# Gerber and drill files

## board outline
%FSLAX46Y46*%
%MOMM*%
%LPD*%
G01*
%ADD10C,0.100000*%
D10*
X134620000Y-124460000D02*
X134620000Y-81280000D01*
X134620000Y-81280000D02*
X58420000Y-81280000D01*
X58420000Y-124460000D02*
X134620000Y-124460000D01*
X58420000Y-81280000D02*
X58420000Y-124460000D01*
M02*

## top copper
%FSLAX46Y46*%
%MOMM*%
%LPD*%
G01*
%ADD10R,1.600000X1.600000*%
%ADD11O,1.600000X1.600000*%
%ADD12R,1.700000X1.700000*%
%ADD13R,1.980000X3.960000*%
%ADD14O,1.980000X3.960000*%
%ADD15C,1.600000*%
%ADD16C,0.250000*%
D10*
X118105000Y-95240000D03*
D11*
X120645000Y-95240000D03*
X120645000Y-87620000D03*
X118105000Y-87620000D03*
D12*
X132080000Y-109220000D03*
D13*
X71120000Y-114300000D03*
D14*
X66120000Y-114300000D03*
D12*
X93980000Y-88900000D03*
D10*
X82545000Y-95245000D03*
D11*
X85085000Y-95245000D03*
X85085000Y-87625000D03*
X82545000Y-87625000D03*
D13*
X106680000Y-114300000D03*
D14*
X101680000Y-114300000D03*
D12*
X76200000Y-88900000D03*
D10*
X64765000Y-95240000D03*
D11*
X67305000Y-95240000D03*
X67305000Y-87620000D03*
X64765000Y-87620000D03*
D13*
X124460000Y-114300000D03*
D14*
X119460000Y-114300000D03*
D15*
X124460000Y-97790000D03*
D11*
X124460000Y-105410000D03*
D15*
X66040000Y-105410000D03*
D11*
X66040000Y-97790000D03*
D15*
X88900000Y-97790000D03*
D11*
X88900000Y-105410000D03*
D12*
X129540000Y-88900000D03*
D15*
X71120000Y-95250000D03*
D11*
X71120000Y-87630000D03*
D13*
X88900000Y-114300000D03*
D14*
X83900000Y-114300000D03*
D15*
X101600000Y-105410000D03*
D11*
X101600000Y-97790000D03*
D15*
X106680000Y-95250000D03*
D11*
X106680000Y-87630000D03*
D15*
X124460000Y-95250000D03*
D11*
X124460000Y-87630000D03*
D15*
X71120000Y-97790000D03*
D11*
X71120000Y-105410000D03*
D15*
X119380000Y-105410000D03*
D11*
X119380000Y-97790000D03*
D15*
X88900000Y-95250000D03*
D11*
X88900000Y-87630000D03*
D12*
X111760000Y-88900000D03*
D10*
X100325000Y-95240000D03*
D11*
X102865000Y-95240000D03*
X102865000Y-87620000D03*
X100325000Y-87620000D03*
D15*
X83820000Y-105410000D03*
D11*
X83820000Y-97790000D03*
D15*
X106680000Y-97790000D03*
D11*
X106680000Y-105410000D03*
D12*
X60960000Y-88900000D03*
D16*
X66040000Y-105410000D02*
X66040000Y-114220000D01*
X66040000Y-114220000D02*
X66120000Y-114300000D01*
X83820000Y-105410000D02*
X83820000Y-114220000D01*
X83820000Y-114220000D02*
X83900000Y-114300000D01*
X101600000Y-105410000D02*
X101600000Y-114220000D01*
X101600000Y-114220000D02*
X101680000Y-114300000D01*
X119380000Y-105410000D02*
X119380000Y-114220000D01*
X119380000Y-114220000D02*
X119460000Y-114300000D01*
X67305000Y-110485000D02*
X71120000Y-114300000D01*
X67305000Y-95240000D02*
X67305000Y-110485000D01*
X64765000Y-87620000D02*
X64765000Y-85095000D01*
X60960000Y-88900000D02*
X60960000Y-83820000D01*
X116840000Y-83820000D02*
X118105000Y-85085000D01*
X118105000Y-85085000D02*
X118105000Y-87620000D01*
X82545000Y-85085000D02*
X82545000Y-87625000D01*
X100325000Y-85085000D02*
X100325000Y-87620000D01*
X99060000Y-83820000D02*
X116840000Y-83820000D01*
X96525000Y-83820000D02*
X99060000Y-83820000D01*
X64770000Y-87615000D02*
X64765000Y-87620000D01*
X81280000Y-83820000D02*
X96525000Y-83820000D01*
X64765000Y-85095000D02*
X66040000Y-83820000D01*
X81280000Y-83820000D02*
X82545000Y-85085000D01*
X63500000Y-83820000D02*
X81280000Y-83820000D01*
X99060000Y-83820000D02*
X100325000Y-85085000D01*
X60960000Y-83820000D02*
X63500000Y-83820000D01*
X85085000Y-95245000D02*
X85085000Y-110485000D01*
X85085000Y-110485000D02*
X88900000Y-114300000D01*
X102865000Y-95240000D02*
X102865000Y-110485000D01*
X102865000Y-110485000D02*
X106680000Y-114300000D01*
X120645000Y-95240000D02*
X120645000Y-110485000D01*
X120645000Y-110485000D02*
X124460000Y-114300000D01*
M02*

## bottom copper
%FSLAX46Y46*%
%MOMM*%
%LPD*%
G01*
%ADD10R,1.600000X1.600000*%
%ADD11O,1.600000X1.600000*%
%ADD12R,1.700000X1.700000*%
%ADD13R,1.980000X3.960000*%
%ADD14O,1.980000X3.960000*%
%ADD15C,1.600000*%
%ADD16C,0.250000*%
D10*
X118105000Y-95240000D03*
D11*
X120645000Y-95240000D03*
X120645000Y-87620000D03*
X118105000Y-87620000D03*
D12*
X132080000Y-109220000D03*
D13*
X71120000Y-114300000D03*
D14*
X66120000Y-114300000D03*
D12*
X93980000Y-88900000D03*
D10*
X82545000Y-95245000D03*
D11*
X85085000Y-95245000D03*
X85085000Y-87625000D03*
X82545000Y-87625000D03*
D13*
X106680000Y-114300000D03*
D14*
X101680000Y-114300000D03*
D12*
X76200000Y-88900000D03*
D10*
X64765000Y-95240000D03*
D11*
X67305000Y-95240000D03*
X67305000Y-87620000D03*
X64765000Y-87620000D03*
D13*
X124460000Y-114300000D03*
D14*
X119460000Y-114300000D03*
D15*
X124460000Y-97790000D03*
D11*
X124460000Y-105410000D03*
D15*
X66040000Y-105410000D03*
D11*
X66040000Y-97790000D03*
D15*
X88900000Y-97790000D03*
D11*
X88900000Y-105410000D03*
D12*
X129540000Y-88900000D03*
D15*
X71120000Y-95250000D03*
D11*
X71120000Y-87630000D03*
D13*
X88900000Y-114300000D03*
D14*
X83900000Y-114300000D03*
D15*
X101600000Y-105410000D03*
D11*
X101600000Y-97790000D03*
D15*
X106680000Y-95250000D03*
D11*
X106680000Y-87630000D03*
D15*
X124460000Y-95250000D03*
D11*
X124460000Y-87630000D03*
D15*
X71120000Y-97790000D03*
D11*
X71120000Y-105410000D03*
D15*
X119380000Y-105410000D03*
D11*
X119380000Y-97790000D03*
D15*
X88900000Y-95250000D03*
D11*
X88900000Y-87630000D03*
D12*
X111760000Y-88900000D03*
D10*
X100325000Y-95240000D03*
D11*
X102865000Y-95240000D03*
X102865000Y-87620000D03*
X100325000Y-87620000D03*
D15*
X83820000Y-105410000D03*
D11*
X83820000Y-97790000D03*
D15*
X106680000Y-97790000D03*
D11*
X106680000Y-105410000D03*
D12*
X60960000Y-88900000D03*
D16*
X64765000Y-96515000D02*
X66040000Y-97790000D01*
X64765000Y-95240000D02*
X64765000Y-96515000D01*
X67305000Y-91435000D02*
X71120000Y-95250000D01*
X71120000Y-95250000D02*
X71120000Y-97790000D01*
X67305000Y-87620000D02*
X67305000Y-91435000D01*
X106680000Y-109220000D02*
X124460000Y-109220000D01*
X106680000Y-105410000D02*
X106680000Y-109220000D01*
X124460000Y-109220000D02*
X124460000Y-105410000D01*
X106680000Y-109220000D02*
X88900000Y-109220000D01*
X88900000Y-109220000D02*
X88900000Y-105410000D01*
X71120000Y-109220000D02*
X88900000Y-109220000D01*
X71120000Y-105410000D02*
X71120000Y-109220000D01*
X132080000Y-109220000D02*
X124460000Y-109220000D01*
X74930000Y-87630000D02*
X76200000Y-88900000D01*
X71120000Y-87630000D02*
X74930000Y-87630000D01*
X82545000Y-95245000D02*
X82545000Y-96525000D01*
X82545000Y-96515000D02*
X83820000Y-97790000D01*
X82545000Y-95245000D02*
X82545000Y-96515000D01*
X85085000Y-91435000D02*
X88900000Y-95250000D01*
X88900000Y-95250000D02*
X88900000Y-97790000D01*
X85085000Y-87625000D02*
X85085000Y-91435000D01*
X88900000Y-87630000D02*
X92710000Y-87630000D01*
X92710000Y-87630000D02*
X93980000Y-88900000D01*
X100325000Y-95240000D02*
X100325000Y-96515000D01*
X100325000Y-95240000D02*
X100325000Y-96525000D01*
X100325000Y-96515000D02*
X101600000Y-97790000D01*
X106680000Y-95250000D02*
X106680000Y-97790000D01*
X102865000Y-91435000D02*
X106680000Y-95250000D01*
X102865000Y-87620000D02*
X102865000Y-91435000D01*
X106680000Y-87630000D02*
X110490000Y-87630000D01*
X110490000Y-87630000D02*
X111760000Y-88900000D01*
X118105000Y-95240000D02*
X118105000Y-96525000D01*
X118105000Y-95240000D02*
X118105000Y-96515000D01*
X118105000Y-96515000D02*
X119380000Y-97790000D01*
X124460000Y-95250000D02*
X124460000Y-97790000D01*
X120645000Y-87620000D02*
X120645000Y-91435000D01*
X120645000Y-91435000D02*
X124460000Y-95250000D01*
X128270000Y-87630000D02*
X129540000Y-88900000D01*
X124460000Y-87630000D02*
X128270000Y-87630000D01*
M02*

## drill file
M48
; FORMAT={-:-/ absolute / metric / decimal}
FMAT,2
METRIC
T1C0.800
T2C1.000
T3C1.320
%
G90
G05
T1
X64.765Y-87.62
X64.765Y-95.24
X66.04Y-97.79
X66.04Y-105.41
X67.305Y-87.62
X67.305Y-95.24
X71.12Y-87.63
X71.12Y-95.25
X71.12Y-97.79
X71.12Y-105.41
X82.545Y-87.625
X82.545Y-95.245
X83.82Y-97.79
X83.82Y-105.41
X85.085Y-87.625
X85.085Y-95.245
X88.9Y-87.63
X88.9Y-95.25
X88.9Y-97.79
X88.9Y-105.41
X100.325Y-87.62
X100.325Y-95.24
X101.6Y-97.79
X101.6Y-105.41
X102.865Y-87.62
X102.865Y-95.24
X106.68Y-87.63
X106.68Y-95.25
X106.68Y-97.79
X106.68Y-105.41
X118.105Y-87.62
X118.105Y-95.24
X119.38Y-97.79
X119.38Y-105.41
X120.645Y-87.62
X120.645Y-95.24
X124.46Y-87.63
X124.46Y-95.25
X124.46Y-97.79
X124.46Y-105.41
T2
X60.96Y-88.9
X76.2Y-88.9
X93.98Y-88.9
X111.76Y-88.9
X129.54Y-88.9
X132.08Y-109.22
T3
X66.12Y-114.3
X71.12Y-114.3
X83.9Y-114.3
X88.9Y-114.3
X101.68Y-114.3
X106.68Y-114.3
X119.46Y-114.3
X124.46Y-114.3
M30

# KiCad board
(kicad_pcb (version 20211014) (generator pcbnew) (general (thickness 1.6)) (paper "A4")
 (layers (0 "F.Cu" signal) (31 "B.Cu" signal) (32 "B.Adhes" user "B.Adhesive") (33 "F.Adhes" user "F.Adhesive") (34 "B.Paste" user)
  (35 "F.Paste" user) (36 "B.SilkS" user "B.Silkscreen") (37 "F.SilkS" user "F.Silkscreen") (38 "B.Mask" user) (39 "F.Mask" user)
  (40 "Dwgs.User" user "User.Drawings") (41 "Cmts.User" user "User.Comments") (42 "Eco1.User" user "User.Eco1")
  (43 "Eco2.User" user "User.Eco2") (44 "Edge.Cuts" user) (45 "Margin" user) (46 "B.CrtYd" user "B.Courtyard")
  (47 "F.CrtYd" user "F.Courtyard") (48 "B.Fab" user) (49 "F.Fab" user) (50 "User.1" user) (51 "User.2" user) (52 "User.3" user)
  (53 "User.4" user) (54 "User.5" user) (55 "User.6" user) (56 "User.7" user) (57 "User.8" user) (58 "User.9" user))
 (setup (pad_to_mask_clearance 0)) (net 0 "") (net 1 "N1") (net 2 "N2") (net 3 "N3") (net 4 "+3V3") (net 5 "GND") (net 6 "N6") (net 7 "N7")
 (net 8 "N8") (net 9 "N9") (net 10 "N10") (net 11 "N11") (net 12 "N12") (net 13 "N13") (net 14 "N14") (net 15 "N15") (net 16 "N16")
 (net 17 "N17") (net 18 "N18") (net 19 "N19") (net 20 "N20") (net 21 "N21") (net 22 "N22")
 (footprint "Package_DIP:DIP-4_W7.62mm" (layer "F.Cu") (at 118.105 95.24 90)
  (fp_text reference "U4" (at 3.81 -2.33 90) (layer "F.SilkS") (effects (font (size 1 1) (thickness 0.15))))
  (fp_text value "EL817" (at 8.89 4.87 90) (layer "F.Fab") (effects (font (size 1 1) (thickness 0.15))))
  (pad "1" thru_hole rect (at 0 0 90) (size 1.6 1.6) (drill 0.8) (layers *.Cu *.Mask) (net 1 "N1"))
  (pad "2" thru_hole oval (at 0 2.54 90) (size 1.6 1.6) (drill 0.8) (layers *.Cu *.Mask) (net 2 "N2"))
  (pad "3" thru_hole oval (at 7.62 2.54 90) (size 1.6 1.6) (drill 0.8) (layers *.Cu *.Mask) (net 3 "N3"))
  (pad "4" thru_hole oval (at 7.62 0 90) (size 1.6 1.6) (drill 0.8) (layers *.Cu *.Mask) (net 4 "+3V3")))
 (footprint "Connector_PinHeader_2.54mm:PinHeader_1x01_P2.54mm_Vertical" (layer "F.Cu") (at 132.08 109.22)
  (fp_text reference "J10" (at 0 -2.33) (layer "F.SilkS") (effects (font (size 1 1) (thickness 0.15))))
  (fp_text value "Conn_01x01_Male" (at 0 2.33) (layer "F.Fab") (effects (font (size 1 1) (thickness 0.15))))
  (pad "1" thru_hole rect (at 0 0) (size 1.7 1.7) (drill 1) (layers *.Cu *.Mask) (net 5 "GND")))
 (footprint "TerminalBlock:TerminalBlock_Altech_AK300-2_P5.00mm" (layer "F.Cu") (at 71.12 114.3 180)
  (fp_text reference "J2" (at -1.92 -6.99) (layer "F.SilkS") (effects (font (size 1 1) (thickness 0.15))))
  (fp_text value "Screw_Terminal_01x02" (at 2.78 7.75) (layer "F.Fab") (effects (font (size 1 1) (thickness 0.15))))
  (pad "1" thru_hole rect (at 0 0 180) (size 1.98 3.96) (drill 1.32) (layers *.Cu *.Mask) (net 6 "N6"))
  (pad "2" thru_hole oval (at 5 0 180) (size 1.98 3.96) (drill 1.32) (layers *.Cu *.Mask) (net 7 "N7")))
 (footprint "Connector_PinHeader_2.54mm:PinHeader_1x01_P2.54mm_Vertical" (layer "F.Cu") (at 93.98 88.9)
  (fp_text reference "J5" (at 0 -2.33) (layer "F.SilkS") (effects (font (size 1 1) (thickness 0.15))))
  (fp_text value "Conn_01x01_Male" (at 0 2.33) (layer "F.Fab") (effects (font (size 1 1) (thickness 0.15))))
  (pad "1" thru_hole rect (at 0 0) (size 1.7 1.7) (drill 1) (layers *.Cu *.Mask) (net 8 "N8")))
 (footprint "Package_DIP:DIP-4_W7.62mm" (layer "F.Cu") (at 82.545 95.245 90)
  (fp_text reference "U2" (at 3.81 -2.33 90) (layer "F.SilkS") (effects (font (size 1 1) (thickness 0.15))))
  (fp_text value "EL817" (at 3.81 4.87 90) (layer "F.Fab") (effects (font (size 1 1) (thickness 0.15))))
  (pad "1" thru_hole rect (at 0 0 90) (size 1.6 1.6) (drill 0.8) (layers *.Cu *.Mask) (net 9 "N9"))
  (pad "2" thru_hole oval (at 0 2.54 90) (size 1.6 1.6) (drill 0.8) (layers *.Cu *.Mask) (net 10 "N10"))
  (pad "3" thru_hole oval (at 7.62 2.54 90) (size 1.6 1.6) (drill 0.8) (layers *.Cu *.Mask) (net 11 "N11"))
  (pad "4" thru_hole oval (at 7.62 0 90) (size 1.6 1.6) (drill 0.8) (layers *.Cu *.Mask) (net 4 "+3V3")))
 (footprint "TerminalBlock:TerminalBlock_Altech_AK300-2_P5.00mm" (layer "F.Cu") (at 106.68 114.3 180)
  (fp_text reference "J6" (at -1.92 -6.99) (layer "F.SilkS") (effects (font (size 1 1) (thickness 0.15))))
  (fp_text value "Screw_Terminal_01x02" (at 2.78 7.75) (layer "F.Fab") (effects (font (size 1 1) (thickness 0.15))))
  (pad "1" thru_hole rect (at 0 0 180) (size 1.98 3.96) (drill 1.32) (layers *.Cu *.Mask) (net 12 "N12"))
  (pad "2" thru_hole oval (at 5 0 180) (size 1.98 3.96) (drill 1.32) (layers *.Cu *.Mask) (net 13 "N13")))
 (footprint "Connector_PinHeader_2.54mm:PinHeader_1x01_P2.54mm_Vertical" (layer "F.Cu") (at 76.2 88.9)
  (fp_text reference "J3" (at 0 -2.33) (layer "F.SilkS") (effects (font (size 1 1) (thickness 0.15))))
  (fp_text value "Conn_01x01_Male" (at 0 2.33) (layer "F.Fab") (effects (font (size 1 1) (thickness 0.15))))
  (pad "1" thru_hole rect (at 0 0) (size 1.7 1.7) (drill 1) (layers *.Cu *.Mask) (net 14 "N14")))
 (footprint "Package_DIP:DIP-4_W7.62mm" (layer "F.Cu") (at 64.765 95.24 90)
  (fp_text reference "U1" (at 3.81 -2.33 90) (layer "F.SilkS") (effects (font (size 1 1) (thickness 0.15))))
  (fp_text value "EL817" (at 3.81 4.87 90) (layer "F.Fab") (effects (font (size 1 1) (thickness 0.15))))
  (pad "1" thru_hole rect (at 0 0 90) (size 1.6 1.6) (drill 0.8) (layers *.Cu *.Mask) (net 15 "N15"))
  (pad "2" thru_hole oval (at 0 2.54 90) (size 1.6 1.6) (drill 0.8) (layers *.Cu *.Mask) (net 6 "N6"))
  (pad "3" thru_hole oval (at 7.62 2.54 90) (size 1.6 1.6) (drill 0.8) (layers *.Cu *.Mask) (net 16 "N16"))
  (pad "4" thru_hole oval (at 7.62 0 90) (size 1.6 1.6) (drill 0.8) (layers *.Cu *.Mask) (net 4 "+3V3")))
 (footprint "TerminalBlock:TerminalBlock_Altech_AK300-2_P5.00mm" (layer "F.Cu") (at 124.46 114.3 180)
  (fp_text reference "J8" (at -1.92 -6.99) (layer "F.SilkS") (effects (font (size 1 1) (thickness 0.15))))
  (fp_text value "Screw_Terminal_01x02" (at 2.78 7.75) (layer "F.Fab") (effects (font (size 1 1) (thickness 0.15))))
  (pad "1" thru_hole rect (at 0 0 180) (size 1.98 3.96) (drill 1.32) (layers *.Cu *.Mask) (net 2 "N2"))
  (pad "2" thru_hole oval (at 5 0 180) (size 1.98 3.96) (drill 1.32) (layers *.Cu *.Mask) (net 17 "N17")))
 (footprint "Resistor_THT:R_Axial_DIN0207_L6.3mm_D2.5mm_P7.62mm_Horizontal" (layer "F.Cu") (at 124.46 97.79 -90)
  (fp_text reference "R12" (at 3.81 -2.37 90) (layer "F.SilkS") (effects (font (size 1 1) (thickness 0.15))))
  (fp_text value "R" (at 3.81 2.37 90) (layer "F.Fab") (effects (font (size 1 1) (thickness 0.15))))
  (pad "1" thru_hole circle (at 0 0 270) (size 1.6 1.6) (drill 0.8) (layers *.Cu *.Mask) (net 3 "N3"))
  (pad "2" thru_hole oval (at 7.62 0 270) (size 1.6 1.6) (drill 0.8) (layers *.Cu *.Mask) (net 5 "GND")))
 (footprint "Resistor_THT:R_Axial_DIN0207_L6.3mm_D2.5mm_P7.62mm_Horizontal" (layer "F.Cu") (at 66.04 105.41 90)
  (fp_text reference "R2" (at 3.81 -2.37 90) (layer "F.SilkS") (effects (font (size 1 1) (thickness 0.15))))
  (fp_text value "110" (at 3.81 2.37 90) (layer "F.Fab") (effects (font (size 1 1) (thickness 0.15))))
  (pad "1" thru_hole circle (at 0 0 90) (size 1.6 1.6) (drill 0.8) (layers *.Cu *.Mask) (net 7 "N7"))
  (pad "2" thru_hole oval (at 7.62 0 90) (size 1.6 1.6) (drill 0.8) (layers *.Cu *.Mask) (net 15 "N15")))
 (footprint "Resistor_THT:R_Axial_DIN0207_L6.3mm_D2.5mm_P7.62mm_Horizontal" (layer "F.Cu") (at 88.9 97.79 -90)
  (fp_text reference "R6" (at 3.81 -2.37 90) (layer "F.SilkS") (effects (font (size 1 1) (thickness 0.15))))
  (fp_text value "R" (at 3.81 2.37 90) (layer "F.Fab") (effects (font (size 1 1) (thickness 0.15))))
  (pad "1" thru_hole circle (at 0 0 270) (size 1.6 1.6) (drill 0.8) (layers *.Cu *.Mask) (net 11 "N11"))
  (pad "2" thru_hole oval (at 7.62 0 270) (size 1.6 1.6) (drill 0.8) (layers *.Cu *.Mask) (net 5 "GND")))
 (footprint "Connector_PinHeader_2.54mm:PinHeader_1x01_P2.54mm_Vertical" (layer "F.Cu") (at 129.54 88.9)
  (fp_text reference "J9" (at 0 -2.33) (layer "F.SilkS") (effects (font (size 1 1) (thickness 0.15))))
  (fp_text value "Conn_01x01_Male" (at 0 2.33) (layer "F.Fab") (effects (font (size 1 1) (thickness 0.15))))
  (pad "1" thru_hole rect (at 0 0) (size 1.7 1.7) (drill 1) (layers *.Cu *.Mask) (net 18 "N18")))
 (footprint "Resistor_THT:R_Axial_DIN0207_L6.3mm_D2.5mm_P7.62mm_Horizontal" (layer "F.Cu") (at 71.12 95.25 90)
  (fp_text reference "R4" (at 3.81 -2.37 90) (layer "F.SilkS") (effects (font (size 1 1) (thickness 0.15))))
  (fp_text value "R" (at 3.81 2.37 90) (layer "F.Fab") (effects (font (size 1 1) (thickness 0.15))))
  (pad "1" thru_hole circle (at 0 0 90) (size 1.6 1.6) (drill 0.8) (layers *.Cu *.Mask) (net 16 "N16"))
  (pad "2" thru_hole oval (at 7.62 0 90) (size 1.6 1.6) (drill 0.8) (layers *.Cu *.Mask) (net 14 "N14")))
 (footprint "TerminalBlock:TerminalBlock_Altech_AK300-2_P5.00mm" (layer "F.Cu") (at 88.9 114.3 180)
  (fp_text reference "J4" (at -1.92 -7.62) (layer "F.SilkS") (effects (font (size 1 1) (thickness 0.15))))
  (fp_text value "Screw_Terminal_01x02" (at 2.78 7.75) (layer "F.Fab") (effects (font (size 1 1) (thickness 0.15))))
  (pad "1" thru_hole rect (at 0 0 180) (size 1.98 3.96) (drill 1.32) (layers *.Cu *.Mask) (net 10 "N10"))
  (pad "2" thru_hole oval (at 5 0 180) (size 1.98 3.96) (drill 1.32) (layers *.Cu *.Mask) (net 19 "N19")))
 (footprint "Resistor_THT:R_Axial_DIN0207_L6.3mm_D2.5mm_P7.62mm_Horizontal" (layer "F.Cu") (at 101.6 105.41 90)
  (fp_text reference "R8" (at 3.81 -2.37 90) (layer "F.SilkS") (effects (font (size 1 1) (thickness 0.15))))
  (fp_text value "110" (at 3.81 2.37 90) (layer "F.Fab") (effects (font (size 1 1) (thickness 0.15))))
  (pad "1" thru_hole circle (at 0 0 90) (size 1.6 1.6) (drill 0.8) (layers *.Cu *.Mask) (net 13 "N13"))
  (pad "2" thru_hole oval (at 7.62 0 90) (size 1.6 1.6) (drill 0.8) (layers *.Cu *.Mask) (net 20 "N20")))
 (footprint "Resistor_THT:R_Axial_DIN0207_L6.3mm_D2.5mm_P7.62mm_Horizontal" (layer "F.Cu") (at 106.68 95.25 90)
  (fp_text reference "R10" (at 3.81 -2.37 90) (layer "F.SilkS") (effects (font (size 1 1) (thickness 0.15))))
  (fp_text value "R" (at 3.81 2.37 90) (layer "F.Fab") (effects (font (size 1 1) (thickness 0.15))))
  (pad "1" thru_hole circle (at 0 0 90) (size 1.6 1.6) (drill 0.8) (layers *.Cu *.Mask) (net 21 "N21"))
  (pad "2" thru_hole oval (at 7.62 0 90) (size 1.6 1.6) (drill 0.8) (layers *.Cu *.Mask) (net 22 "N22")))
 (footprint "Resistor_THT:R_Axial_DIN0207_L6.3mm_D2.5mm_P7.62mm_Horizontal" (layer "F.Cu") (at 124.46 95.25 90)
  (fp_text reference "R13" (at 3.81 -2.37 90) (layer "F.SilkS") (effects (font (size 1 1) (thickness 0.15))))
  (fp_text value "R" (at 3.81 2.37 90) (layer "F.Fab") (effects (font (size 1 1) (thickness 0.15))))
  (pad "1" thru_hole circle (at 0 0 90) (size 1.6 1.6) (drill 0.8) (layers *.Cu *.Mask) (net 3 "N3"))
  (pad "2" thru_hole oval (at 7.62 0 90) (size 1.6 1.6) (drill 0.8) (layers *.Cu *.Mask) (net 18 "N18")))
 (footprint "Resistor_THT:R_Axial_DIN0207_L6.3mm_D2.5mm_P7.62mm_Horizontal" (layer "F.Cu") (at 71.12 97.79 -90)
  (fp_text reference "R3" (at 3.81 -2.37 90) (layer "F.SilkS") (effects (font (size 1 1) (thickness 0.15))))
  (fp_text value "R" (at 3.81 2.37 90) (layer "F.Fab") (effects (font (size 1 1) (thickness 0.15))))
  (pad "1" thru_hole circle (at 0 0 270) (size 1.6 1.6) (drill 0.8) (layers *.Cu *.Mask) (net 16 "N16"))
  (pad "2" thru_hole oval (at 7.62 0 270) (size 1.6 1.6) (drill 0.8) (layers *.Cu *.Mask) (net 5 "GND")))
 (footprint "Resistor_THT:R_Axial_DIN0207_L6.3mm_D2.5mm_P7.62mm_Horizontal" (layer "F.Cu") (at 119.38 105.41 90)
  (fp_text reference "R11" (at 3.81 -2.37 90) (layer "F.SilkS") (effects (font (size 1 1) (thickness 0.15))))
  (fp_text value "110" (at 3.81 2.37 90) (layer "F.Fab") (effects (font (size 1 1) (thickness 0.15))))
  (pad "1" thru_hole circle (at 0 0 90) (size 1.6 1.6) (drill 0.8) (layers *.Cu *.Mask) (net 17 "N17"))
  (pad "2" thru_hole oval (at 7.62 0 90) (size 1.6 1.6) (drill 0.8) (layers *.Cu *.Mask) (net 1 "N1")))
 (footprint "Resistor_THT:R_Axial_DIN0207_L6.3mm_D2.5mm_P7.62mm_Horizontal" (layer "F.Cu") (at 88.9 95.25 90)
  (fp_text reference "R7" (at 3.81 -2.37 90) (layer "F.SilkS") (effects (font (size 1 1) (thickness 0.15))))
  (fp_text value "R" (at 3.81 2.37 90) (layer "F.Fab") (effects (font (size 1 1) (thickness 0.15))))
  (pad "1" thru_hole circle (at 0 0 90) (size 1.6 1.6) (drill 0.8) (layers *.Cu *.Mask) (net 11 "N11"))
  (pad "2" thru_hole oval (at 7.62 0 90) (size 1.6 1.6) (drill 0.8) (layers *.Cu *.Mask) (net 8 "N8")))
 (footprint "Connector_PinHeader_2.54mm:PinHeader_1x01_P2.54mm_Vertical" (layer "F.Cu") (at 111.76 88.9)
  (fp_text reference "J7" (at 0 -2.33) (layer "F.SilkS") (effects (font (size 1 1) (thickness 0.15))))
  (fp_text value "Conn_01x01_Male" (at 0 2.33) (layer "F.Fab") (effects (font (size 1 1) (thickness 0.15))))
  (pad "1" thru_hole rect (at 0 0) (size 1.7 1.7) (drill 1) (layers *.Cu *.Mask) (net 22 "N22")))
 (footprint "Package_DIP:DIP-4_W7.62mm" (layer "F.Cu") (at 100.325 95.24 90)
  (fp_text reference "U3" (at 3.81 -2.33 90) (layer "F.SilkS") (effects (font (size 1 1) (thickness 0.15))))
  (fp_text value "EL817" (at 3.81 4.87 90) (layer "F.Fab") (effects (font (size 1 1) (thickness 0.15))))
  (pad "1" thru_hole rect (at 0 0 90) (size 1.6 1.6) (drill 0.8) (layers *.Cu *.Mask) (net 20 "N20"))
  (pad "2" thru_hole oval (at 0 2.54 90) (size 1.6 1.6) (drill 0.8) (layers *.Cu *.Mask) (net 12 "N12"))
  (pad "3" thru_hole oval (at 7.62 2.54 90) (size 1.6 1.6) (drill 0.8) (layers *.Cu *.Mask) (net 21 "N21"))
  (pad "4" thru_hole oval (at 7.62 0 90) (size 1.6 1.6) (drill 0.8) (layers *.Cu *.Mask) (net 4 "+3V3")))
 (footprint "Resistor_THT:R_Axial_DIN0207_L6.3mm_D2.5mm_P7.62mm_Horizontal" (layer "F.Cu") (at 83.82 105.41 90)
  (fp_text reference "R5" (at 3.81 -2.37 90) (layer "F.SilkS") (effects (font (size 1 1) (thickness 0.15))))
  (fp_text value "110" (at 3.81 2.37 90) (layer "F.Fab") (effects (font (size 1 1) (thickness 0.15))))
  (pad "1" thru_hole circle (at 0 0 90) (size 1.6 1.6) (drill 0.8) (layers *.Cu *.Mask) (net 19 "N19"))
  (pad "2" thru_hole oval (at 7.62 0 90) (size 1.6 1.6) (drill 0.8) (layers *.Cu *.Mask) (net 9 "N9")))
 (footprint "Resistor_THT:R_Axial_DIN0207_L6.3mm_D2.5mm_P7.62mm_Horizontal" (layer "F.Cu") (at 106.68 97.79 -90)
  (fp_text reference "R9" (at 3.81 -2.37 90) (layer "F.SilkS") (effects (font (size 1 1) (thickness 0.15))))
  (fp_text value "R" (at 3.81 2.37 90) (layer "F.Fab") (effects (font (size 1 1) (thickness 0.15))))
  (pad "1" thru_hole circle (at 0 0 270) (size 1.6 1.6) (drill 0.8) (layers *.Cu *.Mask) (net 21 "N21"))
  (pad "2" thru_hole oval (at 7.62 0 270) (size 1.6 1.6) (drill 0.8) (layers *.Cu *.Mask) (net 5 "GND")))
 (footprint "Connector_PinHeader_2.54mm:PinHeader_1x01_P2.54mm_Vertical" (layer "F.Cu") (at 60.96 88.9)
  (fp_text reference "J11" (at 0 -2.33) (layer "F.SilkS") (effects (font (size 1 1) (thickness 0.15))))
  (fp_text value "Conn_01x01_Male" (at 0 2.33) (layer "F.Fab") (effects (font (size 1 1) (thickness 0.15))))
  (pad "1" thru_hole rect (at 0 0) (size 1.7 1.7) (drill 1) (layers *.Cu *.Mask) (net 4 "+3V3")))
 (gr_line (start 134.62 124.46) (end 134.62 81.28) (layer "Edge.Cuts") (width 0.1))
 (gr_line (start 134.62 81.28) (end 58.42 81.28) (layer "Edge.Cuts") (width 0.1))
 (gr_line (start 58.42 124.46) (end 134.62 124.46) (layer "Edge.Cuts") (width 0.1))
 (gr_line (start 58.42 81.28) (end 58.42 124.46) (layer "Edge.Cuts") (width 0.1))
 (segment (start 66.04 105.41) (end 66.04 114.22) (width 0.25) (layer "F.Cu") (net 7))
 (segment (start 66.04 114.22) (end 66.12 114.3) (width 0.25) (layer "F.Cu") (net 7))
 (segment (start 64.765 96.515) (end 66.04 97.79) (width 0.25) (layer "B.Cu") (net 15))
 (segment (start 64.765 95.24) (end 64.765 96.515) (width 0.25) (layer "B.Cu") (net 15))
 (segment (start 67.305 91.435) (end 71.12 95.25) (width 0.25) (layer "B.Cu") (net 16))
 (segment (start 71.12 95.25) (end 71.12 97.79) (width 0.25) (layer "B.Cu") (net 16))
 (segment (start 67.305 87.62) (end 67.305 91.435) (width 0.25) (layer "B.Cu") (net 16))
 (segment (start 106.68 109.22) (end 124.46 109.22) (width 0.25) (layer "B.Cu") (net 5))
 (segment (start 106.68 105.41) (end 106.68 109.22) (width 0.25) (layer "B.Cu") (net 5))
 (segment (start 124.46 109.22) (end 124.46 105.41) (width 0.25) (layer "B.Cu") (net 5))
 (segment (start 106.68 109.22) (end 88.9 109.22) (width 0.25) (layer "B.Cu") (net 5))
 (segment (start 88.9 109.22) (end 88.9 105.41) (width 0.25) (layer "B.Cu") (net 5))
 (segment (start 71.12 109.22) (end 88.9 109.22) (width 0.25) (layer "B.Cu") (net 5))
 (segment (start 71.12 105.41) (end 71.12 109.22) (width 0.25) (layer "B.Cu") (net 5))
 (segment (start 132.08 109.22) (end 124.46 109.22) (width 0.25) (layer "B.Cu") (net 5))
 (segment (start 74.93 87.63) (end 76.2 88.9) (width 0.25) (layer "B.Cu") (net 14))
 (segment (start 71.12 87.63) (end 74.93 87.63) (width 0.25) (layer "B.Cu") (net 14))
 (segment (start 83.82 105.41) (end 83.82 114.22) (width 0.25) (layer "F.Cu") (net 19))
 (segment (start 83.82 114.22) (end 83.9 114.3) (width 0.25) (layer "F.Cu") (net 19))
 (segment (start 82.545 95.245) (end 82.545 96.525) (width 0.25) (layer "B.Cu") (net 9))
 (segment (start 82.545 96.515) (end 83.82 97.79) (width 0.25) (layer "B.Cu") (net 9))
 (segment (start 82.545 95.245) (end 82.545 96.515) (width 0.25) (layer "B.Cu") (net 9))
 (segment (start 85.085 91.435) (end 88.9 95.25) (width 0.25) (layer "B.Cu") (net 11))
 (segment (start 88.9 95.25) (end 88.9 97.79) (width 0.25) (layer "B.Cu") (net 11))
 (segment (start 85.085 87.625) (end 85.085 91.435) (width 0.25) (layer "B.Cu") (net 11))
 (segment (start 88.9 87.63) (end 92.71 87.63) (width 0.25) (layer "B.Cu") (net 8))
 (segment (start 92.71 87.63) (end 93.98 88.9) (width 0.25) (layer "B.Cu") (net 8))
 (segment (start 101.6 105.41) (end 101.6 114.22) (width 0.25) (layer "F.Cu") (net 13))
 (segment (start 101.6 114.22) (end 101.68 114.3) (width 0.25) (layer "F.Cu") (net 13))
 (segment (start 100.325 95.24) (end 100.325 96.515) (width 0.25) (layer "B.Cu") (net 20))
 (segment (start 100.325 95.24) (end 100.325 96.525) (width 0.25) (layer "B.Cu") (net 20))
 (segment (start 100.325 96.515) (end 101.6 97.79) (width 0.25) (layer "B.Cu") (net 20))
 (segment (start 106.68 95.25) (end 106.68 97.79) (width 0.25) (layer "B.Cu") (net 21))
 (segment (start 102.865 91.435) (end 106.68 95.25) (width 0.25) (layer "B.Cu") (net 21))
 (segment (start 102.865 87.62) (end 102.865 91.435) (width 0.25) (layer "B.Cu") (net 21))
 (segment (start 106.68 87.63) (end 110.49 87.63) (width 0.25) (layer "B.Cu") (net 22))
 (segment (start 110.49 87.63) (end 111.76 88.9) (width 0.25) (layer "B.Cu") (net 22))
 (segment (start 119.38 105.41) (end 119.38 114.22) (width 0.25) (layer "F.Cu") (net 17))
 (segment (start 119.38 114.22) (end 119.46 114.3) (width 0.25) (layer "F.Cu") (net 17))
 (segment (start 118.105 95.24) (end 118.105 96.525) (width 0.25) (layer "B.Cu") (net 1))
 (segment (start 118.105 95.24) (end 118.105 96.515) (width 0.25) (layer "B.Cu") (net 1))
 (segment (start 118.105 96.515) (end 119.38 97.79) (width 0.25) (layer "B.Cu") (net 1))
 (segment (start 124.46 95.25) (end 124.46 97.79) (width 0.25) (layer "B.Cu") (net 3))
 (segment (start 120.645 87.62) (end 120.645 91.435) (width 0.25) (layer "B.Cu") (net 3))
 (segment (start 120.645 91.435) (end 124.46 95.25) (width 0.25) (layer "B.Cu") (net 3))
 (segment (start 128.27 87.63) (end 129.54 88.9) (width 0.25) (layer "B.Cu") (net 18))
 (segment (start 124.46 87.63) (end 128.27 87.63) (width 0.25) (layer "B.Cu") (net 18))
 (segment (start 67.305 110.485) (end 71.12 114.3) (width 0.25) (layer "F.Cu") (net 6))
 (segment (start 67.305 95.24) (end 67.305 110.485) (width 0.25) (layer "F.Cu") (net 6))
 (segment (start 64.765 87.62) (end 64.765 85.095) (width 0.25) (layer "F.Cu") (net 4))
 (segment (start 60.96 88.9) (end 60.96 83.82) (width 0.25) (layer "F.Cu") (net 4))
 (segment (start 116.84 83.82) (end 118.105 85.085) (width 0.25) (layer "F.Cu") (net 4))
 (segment (start 118.105 85.085) (end 118.105 87.62) (width 0.25) (layer "F.Cu") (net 4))
 (segment (start 82.545 85.085) (end 82.545 87.625) (width 0.25) (layer "F.Cu") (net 4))
 (segment (start 100.325 85.085) (end 100.325 87.62) (width 0.25) (layer "F.Cu") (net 4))
 (segment (start 99.06 83.82) (end 116.84 83.82) (width 0.25) (layer "F.Cu") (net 4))
 (segment (start 96.525 83.82) (end 99.06 83.82) (width 0.25) (layer "F.Cu") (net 4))
 (segment (start 64.77 87.615) (end 64.765 87.62) (width 0.25) (layer "F.Cu") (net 4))
 (segment (start 81.28 83.82) (end 96.525 83.82) (width 0.25) (layer "F.Cu") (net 4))
 (segment (start 64.765 85.095) (end 66.04 83.82) (width 0.25) (layer "F.Cu") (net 4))
 (segment (start 81.28 83.82) (end 82.545 85.085) (width 0.25) (layer "F.Cu") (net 4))
 (segment (start 63.5 83.82) (end 81.28 83.82) (width 0.25) (layer "F.Cu") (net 4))
 (segment (start 99.06 83.82) (end 100.325 85.085) (width 0.25) (layer "F.Cu") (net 4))
 (segment (start 60.96 83.82) (end 63.5 83.82) (width 0.25) (layer "F.Cu") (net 4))
 (segment (start 85.085 95.245) (end 85.085 110.485) (width 0.25) (layer "F.Cu") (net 10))
 (segment (start 85.085 110.485) (end 88.9 114.3) (width 0.25) (layer "F.Cu") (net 10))
 (segment (start 102.865 95.24) (end 102.865 110.485) (width 0.25) (layer "F.Cu") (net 12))
 (segment (start 102.865 110.485) (end 106.68 114.3) (width 0.25) (layer "F.Cu") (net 12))
 (segment (start 120.645 95.24) (end 120.645 110.485) (width 0.25) (layer "F.Cu") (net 2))
 (segment (start 120.645 110.485) (end 124.46 114.3) (width 0.25) (layer "F.Cu") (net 2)))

